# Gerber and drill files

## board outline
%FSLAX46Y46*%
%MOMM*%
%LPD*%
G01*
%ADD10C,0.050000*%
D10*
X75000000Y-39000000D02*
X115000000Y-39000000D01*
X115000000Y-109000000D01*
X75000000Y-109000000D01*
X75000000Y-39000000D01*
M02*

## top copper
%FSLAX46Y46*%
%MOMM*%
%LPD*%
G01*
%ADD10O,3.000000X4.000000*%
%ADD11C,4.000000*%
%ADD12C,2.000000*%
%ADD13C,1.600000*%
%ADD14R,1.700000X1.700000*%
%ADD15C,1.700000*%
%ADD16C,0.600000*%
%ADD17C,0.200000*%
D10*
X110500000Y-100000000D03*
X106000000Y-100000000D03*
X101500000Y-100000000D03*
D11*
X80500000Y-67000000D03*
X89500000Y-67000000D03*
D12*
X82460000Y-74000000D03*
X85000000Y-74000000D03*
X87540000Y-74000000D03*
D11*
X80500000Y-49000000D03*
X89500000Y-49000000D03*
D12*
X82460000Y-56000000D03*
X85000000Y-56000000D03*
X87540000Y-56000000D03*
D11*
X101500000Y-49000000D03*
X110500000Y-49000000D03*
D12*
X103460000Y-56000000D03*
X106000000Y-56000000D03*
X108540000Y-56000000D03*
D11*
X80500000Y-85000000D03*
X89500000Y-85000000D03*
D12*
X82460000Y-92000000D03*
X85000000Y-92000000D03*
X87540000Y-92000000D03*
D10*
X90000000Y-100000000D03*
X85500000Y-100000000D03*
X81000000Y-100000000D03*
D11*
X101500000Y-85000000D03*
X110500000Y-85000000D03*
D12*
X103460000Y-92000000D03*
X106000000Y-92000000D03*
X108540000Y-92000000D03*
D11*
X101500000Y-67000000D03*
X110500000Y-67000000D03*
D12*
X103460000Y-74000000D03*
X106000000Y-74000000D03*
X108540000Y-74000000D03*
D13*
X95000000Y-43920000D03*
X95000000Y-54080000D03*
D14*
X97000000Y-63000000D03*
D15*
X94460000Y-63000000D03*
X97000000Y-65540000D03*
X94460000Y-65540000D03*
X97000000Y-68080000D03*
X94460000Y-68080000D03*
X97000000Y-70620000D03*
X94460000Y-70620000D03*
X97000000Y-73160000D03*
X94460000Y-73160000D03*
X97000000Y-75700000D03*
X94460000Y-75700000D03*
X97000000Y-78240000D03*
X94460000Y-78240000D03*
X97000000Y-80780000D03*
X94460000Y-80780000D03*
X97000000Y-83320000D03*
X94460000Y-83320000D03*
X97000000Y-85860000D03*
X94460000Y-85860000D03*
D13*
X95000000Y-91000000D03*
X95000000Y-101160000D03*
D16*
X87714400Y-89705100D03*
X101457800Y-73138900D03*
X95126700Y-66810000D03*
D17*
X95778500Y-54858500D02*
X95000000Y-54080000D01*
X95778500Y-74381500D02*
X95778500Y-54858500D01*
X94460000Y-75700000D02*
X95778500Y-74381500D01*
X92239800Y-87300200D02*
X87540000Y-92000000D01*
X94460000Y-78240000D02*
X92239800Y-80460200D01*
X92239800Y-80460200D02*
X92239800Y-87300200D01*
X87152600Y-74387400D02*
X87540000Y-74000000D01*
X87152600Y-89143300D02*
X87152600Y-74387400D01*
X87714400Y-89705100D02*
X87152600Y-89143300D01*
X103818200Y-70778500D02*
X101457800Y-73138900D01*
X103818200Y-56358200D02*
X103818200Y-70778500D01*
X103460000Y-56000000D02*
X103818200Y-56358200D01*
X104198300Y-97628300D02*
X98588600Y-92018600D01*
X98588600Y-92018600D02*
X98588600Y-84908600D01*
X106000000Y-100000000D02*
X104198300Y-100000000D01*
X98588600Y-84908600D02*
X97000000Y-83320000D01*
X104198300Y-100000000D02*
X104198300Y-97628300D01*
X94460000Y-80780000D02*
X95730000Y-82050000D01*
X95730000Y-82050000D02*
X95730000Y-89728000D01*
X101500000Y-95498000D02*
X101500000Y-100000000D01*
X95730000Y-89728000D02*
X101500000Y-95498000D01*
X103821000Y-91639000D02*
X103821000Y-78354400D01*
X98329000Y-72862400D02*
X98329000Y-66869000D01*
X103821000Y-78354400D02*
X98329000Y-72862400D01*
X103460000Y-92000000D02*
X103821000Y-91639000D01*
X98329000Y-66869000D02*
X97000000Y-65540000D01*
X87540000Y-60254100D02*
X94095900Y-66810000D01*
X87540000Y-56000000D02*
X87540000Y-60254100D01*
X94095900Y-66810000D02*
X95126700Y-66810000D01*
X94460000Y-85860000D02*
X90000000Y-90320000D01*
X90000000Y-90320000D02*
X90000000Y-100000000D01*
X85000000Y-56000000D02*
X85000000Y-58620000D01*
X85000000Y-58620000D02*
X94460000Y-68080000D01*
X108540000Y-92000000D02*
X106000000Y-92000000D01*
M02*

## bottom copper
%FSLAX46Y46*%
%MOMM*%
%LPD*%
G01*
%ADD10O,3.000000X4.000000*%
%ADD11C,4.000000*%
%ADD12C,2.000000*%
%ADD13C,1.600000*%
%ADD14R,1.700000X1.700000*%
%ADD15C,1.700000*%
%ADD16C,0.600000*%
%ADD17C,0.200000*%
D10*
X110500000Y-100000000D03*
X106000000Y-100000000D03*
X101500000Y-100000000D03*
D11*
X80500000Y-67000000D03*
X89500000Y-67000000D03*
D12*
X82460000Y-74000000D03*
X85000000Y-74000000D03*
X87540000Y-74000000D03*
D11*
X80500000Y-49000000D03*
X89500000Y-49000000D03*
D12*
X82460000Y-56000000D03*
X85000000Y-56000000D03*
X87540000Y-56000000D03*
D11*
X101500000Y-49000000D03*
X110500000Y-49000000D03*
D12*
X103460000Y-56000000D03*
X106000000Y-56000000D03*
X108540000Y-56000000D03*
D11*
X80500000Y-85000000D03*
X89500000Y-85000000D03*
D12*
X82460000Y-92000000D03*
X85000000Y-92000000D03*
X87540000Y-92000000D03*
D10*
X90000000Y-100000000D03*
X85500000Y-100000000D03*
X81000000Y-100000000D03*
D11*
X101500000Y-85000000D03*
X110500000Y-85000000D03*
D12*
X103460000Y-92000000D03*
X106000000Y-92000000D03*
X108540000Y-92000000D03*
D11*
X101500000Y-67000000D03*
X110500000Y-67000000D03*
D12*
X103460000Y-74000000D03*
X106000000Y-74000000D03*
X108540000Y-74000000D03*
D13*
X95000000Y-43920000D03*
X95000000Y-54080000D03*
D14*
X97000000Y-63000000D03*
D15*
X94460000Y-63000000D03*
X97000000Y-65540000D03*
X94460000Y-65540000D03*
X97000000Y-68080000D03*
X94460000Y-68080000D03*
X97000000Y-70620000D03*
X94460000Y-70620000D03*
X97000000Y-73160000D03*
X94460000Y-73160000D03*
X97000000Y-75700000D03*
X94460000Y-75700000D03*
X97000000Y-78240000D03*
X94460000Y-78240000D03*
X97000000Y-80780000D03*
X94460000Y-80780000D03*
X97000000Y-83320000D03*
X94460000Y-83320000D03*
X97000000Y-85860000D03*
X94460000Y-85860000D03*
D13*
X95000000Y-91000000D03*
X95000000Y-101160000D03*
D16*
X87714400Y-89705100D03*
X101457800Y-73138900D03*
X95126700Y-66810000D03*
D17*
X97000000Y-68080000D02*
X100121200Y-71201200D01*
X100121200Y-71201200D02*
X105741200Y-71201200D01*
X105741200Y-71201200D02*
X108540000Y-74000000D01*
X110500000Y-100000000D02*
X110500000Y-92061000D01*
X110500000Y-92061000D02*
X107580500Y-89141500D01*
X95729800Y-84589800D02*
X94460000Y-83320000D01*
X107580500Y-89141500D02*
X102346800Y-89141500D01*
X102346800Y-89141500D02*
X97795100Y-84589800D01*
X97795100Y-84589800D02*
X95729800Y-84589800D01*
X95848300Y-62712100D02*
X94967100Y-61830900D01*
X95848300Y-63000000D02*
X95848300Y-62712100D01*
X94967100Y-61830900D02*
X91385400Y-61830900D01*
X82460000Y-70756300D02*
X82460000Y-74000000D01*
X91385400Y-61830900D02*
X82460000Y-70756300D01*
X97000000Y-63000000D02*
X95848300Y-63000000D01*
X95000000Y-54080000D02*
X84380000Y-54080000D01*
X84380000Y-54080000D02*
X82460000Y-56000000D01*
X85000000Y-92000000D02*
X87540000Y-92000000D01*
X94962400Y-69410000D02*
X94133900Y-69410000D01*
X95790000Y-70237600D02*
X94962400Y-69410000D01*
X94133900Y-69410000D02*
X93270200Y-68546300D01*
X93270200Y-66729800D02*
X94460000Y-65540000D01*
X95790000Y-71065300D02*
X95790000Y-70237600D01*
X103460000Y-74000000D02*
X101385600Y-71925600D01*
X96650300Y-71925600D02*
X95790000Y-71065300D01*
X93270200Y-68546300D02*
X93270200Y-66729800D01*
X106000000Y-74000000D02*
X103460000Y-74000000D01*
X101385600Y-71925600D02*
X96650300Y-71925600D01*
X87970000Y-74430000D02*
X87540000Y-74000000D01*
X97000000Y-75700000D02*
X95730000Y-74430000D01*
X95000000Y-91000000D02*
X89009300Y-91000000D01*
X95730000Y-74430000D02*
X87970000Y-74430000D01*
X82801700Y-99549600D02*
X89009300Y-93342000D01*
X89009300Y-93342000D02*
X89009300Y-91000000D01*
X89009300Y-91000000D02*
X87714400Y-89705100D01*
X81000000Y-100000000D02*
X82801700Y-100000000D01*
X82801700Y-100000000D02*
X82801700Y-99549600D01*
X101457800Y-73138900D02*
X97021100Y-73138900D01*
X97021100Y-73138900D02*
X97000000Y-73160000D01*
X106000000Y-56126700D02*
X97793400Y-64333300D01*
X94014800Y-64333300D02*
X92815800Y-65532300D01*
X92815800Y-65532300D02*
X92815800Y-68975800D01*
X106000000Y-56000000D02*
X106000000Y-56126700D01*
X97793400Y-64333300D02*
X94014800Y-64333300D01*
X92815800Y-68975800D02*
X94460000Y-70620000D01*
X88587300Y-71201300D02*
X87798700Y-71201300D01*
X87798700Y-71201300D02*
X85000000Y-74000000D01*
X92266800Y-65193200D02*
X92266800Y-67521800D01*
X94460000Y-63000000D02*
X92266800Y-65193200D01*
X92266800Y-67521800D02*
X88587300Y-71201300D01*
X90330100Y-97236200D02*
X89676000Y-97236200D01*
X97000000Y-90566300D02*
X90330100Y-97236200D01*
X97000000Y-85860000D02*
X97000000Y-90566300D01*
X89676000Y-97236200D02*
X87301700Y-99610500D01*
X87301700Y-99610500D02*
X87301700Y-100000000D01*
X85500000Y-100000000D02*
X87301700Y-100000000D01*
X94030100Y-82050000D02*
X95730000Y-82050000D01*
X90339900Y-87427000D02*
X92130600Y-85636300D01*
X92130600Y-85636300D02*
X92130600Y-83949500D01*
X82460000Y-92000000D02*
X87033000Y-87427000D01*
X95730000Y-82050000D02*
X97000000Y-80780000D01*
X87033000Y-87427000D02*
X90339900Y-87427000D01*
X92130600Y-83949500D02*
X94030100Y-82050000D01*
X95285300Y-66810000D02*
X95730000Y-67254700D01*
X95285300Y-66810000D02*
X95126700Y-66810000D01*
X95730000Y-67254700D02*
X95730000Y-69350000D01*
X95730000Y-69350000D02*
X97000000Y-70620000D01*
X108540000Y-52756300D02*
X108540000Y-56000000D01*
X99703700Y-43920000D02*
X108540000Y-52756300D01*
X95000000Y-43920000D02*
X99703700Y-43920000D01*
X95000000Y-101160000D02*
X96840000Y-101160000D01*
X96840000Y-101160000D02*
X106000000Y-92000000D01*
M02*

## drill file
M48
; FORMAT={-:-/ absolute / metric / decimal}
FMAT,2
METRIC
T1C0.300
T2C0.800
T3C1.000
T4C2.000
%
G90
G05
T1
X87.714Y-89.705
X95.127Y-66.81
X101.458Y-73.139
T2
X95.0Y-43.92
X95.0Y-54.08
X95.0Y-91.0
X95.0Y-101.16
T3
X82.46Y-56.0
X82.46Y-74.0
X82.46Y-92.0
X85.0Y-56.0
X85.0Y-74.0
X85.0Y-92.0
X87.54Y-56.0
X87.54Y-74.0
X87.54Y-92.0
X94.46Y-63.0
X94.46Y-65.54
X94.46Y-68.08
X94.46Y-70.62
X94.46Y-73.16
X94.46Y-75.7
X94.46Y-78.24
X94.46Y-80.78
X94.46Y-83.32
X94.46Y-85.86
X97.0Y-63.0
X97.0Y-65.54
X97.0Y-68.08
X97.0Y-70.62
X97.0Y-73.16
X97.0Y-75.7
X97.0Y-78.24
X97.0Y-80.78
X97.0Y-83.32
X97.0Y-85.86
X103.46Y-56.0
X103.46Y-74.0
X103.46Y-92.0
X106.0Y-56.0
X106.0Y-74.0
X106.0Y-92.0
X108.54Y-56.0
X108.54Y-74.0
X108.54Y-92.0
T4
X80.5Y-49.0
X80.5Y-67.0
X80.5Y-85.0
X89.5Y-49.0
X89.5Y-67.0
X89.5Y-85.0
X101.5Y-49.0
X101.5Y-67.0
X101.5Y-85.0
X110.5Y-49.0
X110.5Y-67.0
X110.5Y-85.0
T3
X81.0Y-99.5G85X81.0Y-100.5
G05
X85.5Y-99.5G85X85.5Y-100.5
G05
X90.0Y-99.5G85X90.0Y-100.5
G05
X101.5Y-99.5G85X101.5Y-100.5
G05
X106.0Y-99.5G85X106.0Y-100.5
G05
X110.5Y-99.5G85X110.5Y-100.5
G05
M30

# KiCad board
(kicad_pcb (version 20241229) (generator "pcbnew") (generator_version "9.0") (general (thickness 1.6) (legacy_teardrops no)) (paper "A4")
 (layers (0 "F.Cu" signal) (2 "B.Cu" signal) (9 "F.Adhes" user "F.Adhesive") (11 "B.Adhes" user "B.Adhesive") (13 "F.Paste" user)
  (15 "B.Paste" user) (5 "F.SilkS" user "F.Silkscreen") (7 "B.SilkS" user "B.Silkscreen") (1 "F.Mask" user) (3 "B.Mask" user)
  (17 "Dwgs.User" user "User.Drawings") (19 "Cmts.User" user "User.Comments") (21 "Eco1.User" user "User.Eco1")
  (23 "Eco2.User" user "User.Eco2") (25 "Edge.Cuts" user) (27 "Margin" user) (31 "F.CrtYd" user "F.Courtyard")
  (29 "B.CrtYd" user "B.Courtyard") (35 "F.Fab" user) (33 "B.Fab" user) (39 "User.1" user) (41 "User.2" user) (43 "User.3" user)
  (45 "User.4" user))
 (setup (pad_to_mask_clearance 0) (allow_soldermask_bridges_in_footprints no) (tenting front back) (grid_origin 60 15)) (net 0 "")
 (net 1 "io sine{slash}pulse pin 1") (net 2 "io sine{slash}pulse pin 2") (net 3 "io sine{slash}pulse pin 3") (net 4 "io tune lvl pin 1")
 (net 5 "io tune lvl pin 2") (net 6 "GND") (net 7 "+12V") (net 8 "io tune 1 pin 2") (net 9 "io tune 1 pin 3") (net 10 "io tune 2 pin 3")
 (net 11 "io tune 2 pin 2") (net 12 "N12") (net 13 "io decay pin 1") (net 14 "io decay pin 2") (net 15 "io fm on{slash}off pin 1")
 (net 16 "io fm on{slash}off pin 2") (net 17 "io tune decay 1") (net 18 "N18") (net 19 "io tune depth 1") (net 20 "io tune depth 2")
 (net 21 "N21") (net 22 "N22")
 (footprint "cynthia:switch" (layer "F.Cu") (at 106 100 -90)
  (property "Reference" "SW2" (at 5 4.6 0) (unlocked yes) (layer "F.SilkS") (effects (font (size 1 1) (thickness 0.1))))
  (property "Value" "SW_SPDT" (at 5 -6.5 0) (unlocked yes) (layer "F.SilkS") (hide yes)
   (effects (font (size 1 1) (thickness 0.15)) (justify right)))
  (pad "1" thru_hole oval (at 0 -4.5 270) (size 4 3) (drill oval 2 1) (layers "*.Cu" "*.Mask") (remove_unused_layers no)
   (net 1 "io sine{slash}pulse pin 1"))
  (pad "2" thru_hole oval (at 0 0 270) (size 4 3) (drill oval 2 1) (layers "*.Cu" "*.Mask") (remove_unused_layers no)
   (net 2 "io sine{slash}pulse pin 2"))
  (pad "3" thru_hole oval (at 0 4.5 270) (size 4 3) (drill oval 2 1) (layers "*.Cu" "*.Mask") (remove_unused_layers no)
   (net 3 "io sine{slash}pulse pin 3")))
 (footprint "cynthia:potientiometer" (layer "F.Cu") (at 85 67)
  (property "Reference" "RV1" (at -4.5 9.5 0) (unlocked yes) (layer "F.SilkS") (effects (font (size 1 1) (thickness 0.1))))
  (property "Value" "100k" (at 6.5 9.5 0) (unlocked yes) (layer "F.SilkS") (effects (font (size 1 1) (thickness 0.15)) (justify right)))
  (pad "" thru_hole circle (at -4.5 0) (size 4 4) (drill 2) (layers "*.Cu" "*.Mask") (remove_unused_layers no))
  (pad "" thru_hole circle (at 4.5 0) (size 4 4) (drill 2) (layers "*.Cu" "*.Mask") (remove_unused_layers no))
  (pad "1" thru_hole circle (at -2.54 7) (size 2 2) (drill 1) (layers "*.Cu" "*.Mask") (remove_unused_layers no) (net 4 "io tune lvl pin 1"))
  (pad "2" thru_hole circle (at 0 7) (size 2 2) (drill 1) (layers "*.Cu" "*.Mask") (remove_unused_layers no) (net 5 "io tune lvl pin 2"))
  (pad "3" thru_hole circle (at 2.54 7) (size 2 2) (drill 1) (layers "*.Cu" "*.Mask") (remove_unused_layers no) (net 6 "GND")))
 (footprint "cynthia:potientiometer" (layer "F.Cu") (at 85 49)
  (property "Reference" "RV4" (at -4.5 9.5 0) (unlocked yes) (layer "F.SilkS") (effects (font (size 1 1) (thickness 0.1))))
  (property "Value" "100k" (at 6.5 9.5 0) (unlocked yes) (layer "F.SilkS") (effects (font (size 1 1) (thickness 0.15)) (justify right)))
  (pad "" thru_hole circle (at -4.5 0) (size 4 4) (drill 2) (layers "*.Cu" "*.Mask") (remove_unused_layers no))
  (pad "" thru_hole circle (at 4.5 0) (size 4 4) (drill 2) (layers "*.Cu" "*.Mask") (remove_unused_layers no))
  (pad "1" thru_hole circle (at -2.54 7) (size 2 2) (drill 1) (layers "*.Cu" "*.Mask") (remove_unused_layers no) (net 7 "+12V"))
  (pad "2" thru_hole circle (at 0 7) (size 2 2) (drill 1) (layers "*.Cu" "*.Mask") (remove_unused_layers no) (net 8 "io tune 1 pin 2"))
  (pad "3" thru_hole circle (at 2.54 7) (size 2 2) (drill 1) (layers "*.Cu" "*.Mask") (remove_unused_layers no) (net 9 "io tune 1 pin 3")))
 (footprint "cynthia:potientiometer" (layer "F.Cu") (at 106 49)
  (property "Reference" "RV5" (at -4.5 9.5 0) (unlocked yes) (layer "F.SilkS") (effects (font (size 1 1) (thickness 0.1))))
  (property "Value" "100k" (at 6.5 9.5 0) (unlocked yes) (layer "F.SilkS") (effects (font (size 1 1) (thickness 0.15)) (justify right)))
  (pad "" thru_hole circle (at -4.5 0) (size 4 4) (drill 2) (layers "*.Cu" "*.Mask") (remove_unused_layers no))
  (pad "" thru_hole circle (at 4.5 0) (size 4 4) (drill 2) (layers "*.Cu" "*.Mask") (remove_unused_layers no))
  (pad "1" thru_hole circle (at -2.54 7) (size 2 2) (drill 1) (layers "*.Cu" "*.Mask") (remove_unused_layers no) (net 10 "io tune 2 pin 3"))
  (pad "2" thru_hole circle (at 0 7) (size 2 2) (drill 1) (layers "*.Cu" "*.Mask") (remove_unused_layers no) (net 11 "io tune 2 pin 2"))
  (pad "3" thru_hole circle (at 2.54 7) (size 2 2) (drill 1) (layers "*.Cu" "*.Mask") (remove_unused_layers no) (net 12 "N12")))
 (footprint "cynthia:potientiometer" (layer "F.Cu") (at 85 85)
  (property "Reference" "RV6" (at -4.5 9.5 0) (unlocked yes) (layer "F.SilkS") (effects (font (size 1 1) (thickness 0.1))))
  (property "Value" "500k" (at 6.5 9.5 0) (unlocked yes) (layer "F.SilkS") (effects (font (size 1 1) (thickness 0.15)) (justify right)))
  (pad "" thru_hole circle (at -4.5 0) (size 4 4) (drill 2) (layers "*.Cu" "*.Mask") (remove_unused_layers no))
  (pad "" thru_hole circle (at 4.5 0) (size 4 4) (drill 2) (layers "*.Cu" "*.Mask") (remove_unused_layers no))
  (pad "1" thru_hole circle (at -2.54 7) (size 2 2) (drill 1) (layers "*.Cu" "*.Mask") (remove_unused_layers no) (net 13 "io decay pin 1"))
  (pad "2" thru_hole circle (at 0 7) (size 2 2) (drill 1) (layers "*.Cu" "*.Mask") (remove_unused_layers no) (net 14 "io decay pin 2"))
  (pad "3" thru_hole circle (at 2.54 7) (size 2 2) (drill 1) (layers "*.Cu" "*.Mask") (remove_unused_layers no) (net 14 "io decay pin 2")))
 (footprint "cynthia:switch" (layer "F.Cu") (at 85.5 100 -90)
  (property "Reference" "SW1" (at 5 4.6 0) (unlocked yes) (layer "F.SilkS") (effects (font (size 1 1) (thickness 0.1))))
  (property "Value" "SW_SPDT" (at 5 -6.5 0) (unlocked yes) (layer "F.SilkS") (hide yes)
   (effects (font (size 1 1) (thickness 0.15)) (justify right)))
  (pad "1" thru_hole oval (at 0 -4.5 270) (size 4 3) (drill oval 2 1) (layers "*.Cu" "*.Mask") (remove_unused_layers no)
   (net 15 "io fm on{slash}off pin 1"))
  (pad "2" thru_hole oval (at 0 0 270) (size 4 3) (drill oval 2 1) (layers "*.Cu" "*.Mask") (remove_unused_layers no)
   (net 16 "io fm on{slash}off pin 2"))
  (pad "3" thru_hole oval (at 0 4.5 270) (size 4 3) (drill oval 2 1) (layers "*.Cu" "*.Mask") (remove_unused_layers no) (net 6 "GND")))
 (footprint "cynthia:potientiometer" (layer "F.Cu") (at 106 85)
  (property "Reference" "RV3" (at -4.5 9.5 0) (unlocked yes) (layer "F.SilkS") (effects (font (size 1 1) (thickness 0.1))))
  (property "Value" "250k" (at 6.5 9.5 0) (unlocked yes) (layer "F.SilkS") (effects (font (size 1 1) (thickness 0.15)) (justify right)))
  (pad "" thru_hole circle (at -4.5 0) (size 4 4) (drill 2) (layers "*.Cu" "*.Mask") (remove_unused_layers no))
  (pad "" thru_hole circle (at 4.5 0) (size 4 4) (drill 2) (layers "*.Cu" "*.Mask") (remove_unused_layers no))
  (pad "1" thru_hole circle (at -2.54 7) (size 2 2) (drill 1) (layers "*.Cu" "*.Mask") (remove_unused_layers no) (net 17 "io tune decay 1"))
  (pad "2" thru_hole circle (at 0 7) (size 2 2) (drill 1) (layers "*.Cu" "*.Mask") (remove_unused_layers no) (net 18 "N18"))
  (pad "3" thru_hole circle (at 2.54 7) (size 2 2) (drill 1) (layers "*.Cu" "*.Mask") (remove_unused_layers no) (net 18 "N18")))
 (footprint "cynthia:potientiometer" (layer "F.Cu") (at 106 67)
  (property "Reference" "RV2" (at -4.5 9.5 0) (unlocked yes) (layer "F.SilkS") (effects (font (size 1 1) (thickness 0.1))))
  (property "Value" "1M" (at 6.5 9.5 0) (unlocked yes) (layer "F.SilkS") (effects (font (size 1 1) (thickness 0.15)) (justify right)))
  (pad "" thru_hole circle (at -4.5 0) (size 4 4) (drill 2) (layers "*.Cu" "*.Mask") (remove_unused_layers no))
  (pad "" thru_hole circle (at 4.5 0) (size 4 4) (drill 2) (layers "*.Cu" "*.Mask") (remove_unused_layers no))
  (pad "1" thru_hole circle (at -2.54 7) (size 2 2) (drill 1) (layers "*.Cu" "*.Mask") (remove_unused_layers no) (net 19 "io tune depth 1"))
  (pad "2" thru_hole circle (at 0 7) (size 2 2) (drill 1) (layers "*.Cu" "*.Mask") (remove_unused_layers no) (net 19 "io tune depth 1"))
  (pad "3" thru_hole circle (at 2.54 7) (size 2 2) (drill 1) (layers "*.Cu" "*.Mask") (remove_unused_layers no) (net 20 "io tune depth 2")))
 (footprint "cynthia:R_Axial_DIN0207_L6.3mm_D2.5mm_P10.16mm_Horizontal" (layer "B.Cu") (at 95 43.92 -90)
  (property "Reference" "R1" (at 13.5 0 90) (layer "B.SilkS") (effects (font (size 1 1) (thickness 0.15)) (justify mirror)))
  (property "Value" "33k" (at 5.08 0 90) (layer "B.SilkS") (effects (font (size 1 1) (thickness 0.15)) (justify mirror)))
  (pad "1" thru_hole circle (at 0 0 270) (size 1.6 1.6) (drill 0.8) (layers "*.Cu" "*.Mask") (remove_unused_layers no) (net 12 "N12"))
  (pad "2" thru_hole circle (at 10.16 0 270) (size 1.6 1.6) (drill 0.8) (layers "*.Cu" "*.Mask") (remove_unused_layers no) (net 7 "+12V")))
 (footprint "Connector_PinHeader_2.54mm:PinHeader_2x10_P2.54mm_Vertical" (layer "B.Cu") (at 97 63 180)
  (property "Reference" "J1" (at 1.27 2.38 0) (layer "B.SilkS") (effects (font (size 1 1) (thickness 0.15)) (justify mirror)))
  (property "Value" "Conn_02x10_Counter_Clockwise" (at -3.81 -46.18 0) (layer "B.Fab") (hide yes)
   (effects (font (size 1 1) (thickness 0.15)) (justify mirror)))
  (pad "1" thru_hole rect (at 0 0 180) (size 1.7 1.7) (drill 1) (layers "*.Cu" "*.Mask") (remove_unused_layers no)
   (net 4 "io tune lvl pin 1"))
  (pad "2" thru_hole circle (at 2.54 0 180) (size 1.7 1.7) (drill 1) (layers "*.Cu" "*.Mask") (remove_unused_layers no)
   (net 5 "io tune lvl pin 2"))
  (pad "3" thru_hole circle (at 0 -2.54 180) (size 1.7 1.7) (drill 1) (layers "*.Cu" "*.Mask") (remove_unused_layers no)
   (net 17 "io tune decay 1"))
  (pad "4" thru_hole circle (at 2.54 -2.54 180) (size 1.7 1.7) (drill 1) (layers "*.Cu" "*.Mask") (remove_unused_layers no)
   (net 19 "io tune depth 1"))
  (pad "5" thru_hole circle (at 0 -5.08 180) (size 1.7 1.7) (drill 1) (layers "*.Cu" "*.Mask") (remove_unused_layers no)
   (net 20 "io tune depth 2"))
  (pad "6" thru_hole circle (at 2.54 -5.08 180) (size 1.7 1.7) (drill 1) (layers "*.Cu" "*.Mask") (remove_unused_layers no)
   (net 8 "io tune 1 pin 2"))
  (pad "7" thru_hole circle (at 0 -7.62 180) (size 1.7 1.7) (drill 1) (layers "*.Cu" "*.Mask") (remove_unused_layers no)
   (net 9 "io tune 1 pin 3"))
  (pad "8" thru_hole circle (at 2.54 -7.62 180) (size 1.7 1.7) (drill 1) (layers "*.Cu" "*.Mask") (remove_unused_layers no)
   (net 11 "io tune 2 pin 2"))
  (pad "9" thru_hole circle (at 0 -10.16 180) (size 1.7 1.7) (drill 1) (layers "*.Cu" "*.Mask") (remove_unused_layers no)
   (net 10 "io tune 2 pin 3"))
  (pad "10" thru_hole circle (at 2.54 -10.16 180) (size 1.7 1.7) (drill 1) (layers "*.Cu" "*.Mask") (remove_unused_layers no) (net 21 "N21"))
  (pad "11" thru_hole circle (at 0 -12.7 180) (size 1.7 1.7) (drill 1) (layers "*.Cu" "*.Mask") (remove_unused_layers no) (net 6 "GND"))
  (pad "12" thru_hole circle (at 2.54 -12.7 180) (size 1.7 1.7) (drill 1) (layers "*.Cu" "*.Mask") (remove_unused_layers no) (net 7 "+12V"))
  (pad "13" thru_hole circle (at 0 -15.24 180) (size 1.7 1.7) (drill 1) (layers "*.Cu" "*.Mask") (remove_unused_layers no) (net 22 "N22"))
  (pad "14" thru_hole circle (at 2.54 -15.24 180) (size 1.7 1.7) (drill 1) (layers "*.Cu" "*.Mask") (remove_unused_layers no)
   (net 14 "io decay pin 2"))
  (pad "15" thru_hole circle (at 0 -17.78 180) (size 1.7 1.7) (drill 1) (layers "*.Cu" "*.Mask") (remove_unused_layers no)
   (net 13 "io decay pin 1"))
  (pad "16" thru_hole circle (at 2.54 -17.78 180) (size 1.7 1.7) (drill 1) (layers "*.Cu" "*.Mask") (remove_unused_layers no)
   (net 3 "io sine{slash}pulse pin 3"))
  (pad "17" thru_hole circle (at 0 -20.32 180) (size 1.7 1.7) (drill 1) (layers "*.Cu" "*.Mask") (remove_unused_layers no)
   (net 2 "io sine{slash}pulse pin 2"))
  (pad "18" thru_hole circle (at 2.54 -20.32 180) (size 1.7 1.7) (drill 1) (layers "*.Cu" "*.Mask") (remove_unused_layers no)
   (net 1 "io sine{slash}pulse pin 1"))
  (pad "19" thru_hole circle (at 0 -22.86 180) (size 1.7 1.7) (drill 1) (layers "*.Cu" "*.Mask") (remove_unused_layers no)
   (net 16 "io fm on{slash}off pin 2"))
  (pad "20" thru_hole circle (at 2.54 -22.86 180) (size 1.7 1.7) (drill 1) (layers "*.Cu" "*.Mask") (remove_unused_layers no)
   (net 15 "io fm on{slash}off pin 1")))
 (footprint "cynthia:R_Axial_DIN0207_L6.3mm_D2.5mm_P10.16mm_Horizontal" (layer "B.Cu") (at 95 91 -90)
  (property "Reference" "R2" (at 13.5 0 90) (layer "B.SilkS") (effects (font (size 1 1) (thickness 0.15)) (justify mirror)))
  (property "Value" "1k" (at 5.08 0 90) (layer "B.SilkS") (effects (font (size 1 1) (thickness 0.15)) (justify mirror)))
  (pad "1" thru_hole circle (at 0 0 270) (size 1.6 1.6) (drill 0.8) (layers "*.Cu" "*.Mask") (remove_unused_layers no) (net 6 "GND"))
  (pad "2" thru_hole circle (at 10.16 0 270) (size 1.6 1.6) (drill 0.8) (layers "*.Cu" "*.Mask") (remove_unused_layers no) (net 18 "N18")))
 (gr_rect (start 75 39) (end 115 109) (stroke (width 0.05) (type default)) (fill no) (layer "Edge.Cuts"))
 (segment (start 97 68.08) (end 100.1212 71.2012) (width 0.2) (layer "B.Cu") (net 20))
 (segment (start 100.1212 71.2012) (end 105.7412 71.2012) (width 0.2) (layer "B.Cu") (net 20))
 (segment (start 105.7412 71.2012) (end 108.54 74) (width 0.2) (layer "B.Cu") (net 20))
 (segment (start 110.5 100) (end 110.5 92.061) (width 0.2) (layer "B.Cu") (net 1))
 (segment (start 110.5 92.061) (end 107.5805 89.1415) (width 0.2) (layer "B.Cu") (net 1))
 (segment (start 95.7298 84.5898) (end 94.46 83.32) (width 0.2) (layer "B.Cu") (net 1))
 (segment (start 107.5805 89.1415) (end 102.3468 89.1415) (width 0.2) (layer "B.Cu") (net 1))
 (segment (start 102.3468 89.1415) (end 97.7951 84.5898) (width 0.2) (layer "B.Cu") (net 1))
 (segment (start 97.7951 84.5898) (end 95.7298 84.5898) (width 0.2) (layer "B.Cu") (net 1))
 (segment (start 95.8483 62.7121) (end 94.9671 61.8309) (width 0.2) (layer "B.Cu") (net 4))
 (segment (start 95.8483 63) (end 95.8483 62.7121) (width 0.2) (layer "B.Cu") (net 4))
 (segment (start 94.9671 61.8309) (end 91.3854 61.8309) (width 0.2) (layer "B.Cu") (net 4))
 (segment (start 82.46 70.7563) (end 82.46 74) (width 0.2) (layer "B.Cu") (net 4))
 (segment (start 91.3854 61.8309) (end 82.46 70.7563) (width 0.2) (layer "B.Cu") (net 4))
 (segment (start 97 63) (end 95.8483 63) (width 0.2) (layer "B.Cu") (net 4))
 (segment (start 95.7785 54.8585) (end 95 54.08) (width 0.2) (layer "F.Cu") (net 7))
 (segment (start 95.7785 74.3815) (end 95.7785 54.8585) (width 0.2) (layer "F.Cu") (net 7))
 (segment (start 94.46 75.7) (end 95.7785 74.3815) (width 0.2) (layer "F.Cu") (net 7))
 (segment (start 95 54.08) (end 84.38 54.08) (width 0.2) (layer "B.Cu") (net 7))
 (segment (start 84.38 54.08) (end 82.46 56) (width 0.2) (layer "B.Cu") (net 7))
 (segment (start 92.2398 87.3002) (end 87.54 92) (width 0.2) (layer "F.Cu") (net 14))
 (segment (start 94.46 78.24) (end 92.2398 80.4602) (width 0.2) (layer "F.Cu") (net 14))
 (segment (start 92.2398 80.4602) (end 92.2398 87.3002) (width 0.2) (layer "F.Cu") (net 14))
 (segment (start 85 92) (end 87.54 92) (width 0.2) (layer "B.Cu") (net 14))
 (segment (start 94.9624 69.41) (end 94.1339 69.41) (width 0.2) (layer "B.Cu") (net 19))
 (segment (start 95.79 70.2376) (end 94.9624 69.41) (width 0.2) (layer "B.Cu") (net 19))
 (segment (start 94.1339 69.41) (end 93.2702 68.5463) (width 0.2) (layer "B.Cu") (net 19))
 (segment (start 93.2702 66.7298) (end 94.46 65.54) (width 0.2) (layer "B.Cu") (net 19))
 (segment (start 95.79 71.0653) (end 95.79 70.2376) (width 0.2) (layer "B.Cu") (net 19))
 (segment (start 103.46 74) (end 101.3856 71.9256) (width 0.2) (layer "B.Cu") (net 19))
 (segment (start 96.6503 71.9256) (end 95.79 71.0653) (width 0.2) (layer "B.Cu") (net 19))
 (segment (start 93.2702 68.5463) (end 93.2702 66.7298) (width 0.2) (layer "B.Cu") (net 19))
 (segment (start 106 74) (end 103.46 74) (width 0.2) (layer "B.Cu") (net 19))
 (segment (start 101.3856 71.9256) (end 96.6503 71.9256) (width 0.2) (layer "B.Cu") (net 19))
 (segment (start 87.1526 74.3874) (end 87.54 74) (width 0.2) (layer "F.Cu") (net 6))
 (segment (start 87.1526 89.1433) (end 87.1526 74.3874) (width 0.2) (layer "F.Cu") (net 6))
 (segment (start 87.7144 89.7051) (end 87.1526 89.1433) (width 0.2) (layer "F.Cu") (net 6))
 (via (at 87.7144 89.7051) (size 0.6) (drill 0.3) (layers "F.Cu" "B.Cu") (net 6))
 (segment (start 87.97 74.43) (end 87.54 74) (width 0.2) (layer "B.Cu") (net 6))
 (segment (start 97 75.7) (end 95.73 74.43) (width 0.2) (layer "B.Cu") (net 6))
 (segment (start 95 91) (end 89.0093 91) (width 0.2) (layer "B.Cu") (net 6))
 (segment (start 95.73 74.43) (end 87.97 74.43) (width 0.2) (layer "B.Cu") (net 6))
 (segment (start 82.8017 99.5496) (end 89.0093 93.342) (width 0.2) (layer "B.Cu") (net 6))
 (segment (start 89.0093 93.342) (end 89.0093 91) (width 0.2) (layer "B.Cu") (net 6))
 (segment (start 89.0093 91) (end 87.7144 89.7051) (width 0.2) (layer "B.Cu") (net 6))
 (segment (start 81 100) (end 82.8017 100) (width 0.2) (layer "B.Cu") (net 6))
 (segment (start 82.8017 100) (end 82.8017 99.5496) (width 0.2) (layer "B.Cu") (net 6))
 (segment (start 103.8182 70.7785) (end 101.4578 73.1389) (width 0.2) (layer "F.Cu") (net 10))
 (segment (start 103.8182 56.3582) (end 103.8182 70.7785) (width 0.2) (layer "F.Cu") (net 10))
 (segment (start 103.46 56) (end 103.8182 56.3582) (width 0.2) (layer "F.Cu") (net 10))
 (via (at 101.4578 73.1389) (size 0.6) (drill 0.3) (layers "F.Cu" "B.Cu") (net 10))
 (segment (start 101.4578 73.1389) (end 97.0211 73.1389) (width 0.2) (layer "B.Cu") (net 10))
 (segment (start 97.0211 73.1389) (end 97 73.16) (width 0.2) (layer "B.Cu") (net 10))
 (segment (start 106 56.1267) (end 97.7934 64.3333) (width 0.2) (layer "B.Cu") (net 11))
 (segment (start 94.0148 64.3333) (end 92.8158 65.5323) (width 0.2) (layer "B.Cu") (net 11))
 (segment (start 92.8158 65.5323) (end 92.8158 68.9758) (width 0.2) (layer "B.Cu") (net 11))
 (segment (start 106 56) (end 106 56.1267) (width 0.2) (layer "B.Cu") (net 11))
 (segment (start 97.7934 64.3333) (end 94.0148 64.3333) (width 0.2) (layer "B.Cu") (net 11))
 (segment (start 92.8158 68.9758) (end 94.46 70.62) (width 0.2) (layer "B.Cu") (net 11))
 (segment (start 88.5873 71.2013) (end 87.7987 71.2013) (width 0.2) (layer "B.Cu") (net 5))
 (segment (start 87.7987 71.2013) (end 85 74) (width 0.2) (layer "B.Cu") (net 5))
 (segment (start 92.2668 65.1932) (end 92.2668 67.5218) (width 0.2) (layer "B.Cu") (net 5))
 (segment (start 94.46 63) (end 92.2668 65.1932) (width 0.2) (layer "B.Cu") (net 5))
 (segment (start 92.2668 67.5218) (end 88.5873 71.2013) (width 0.2) (layer "B.Cu") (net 5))
 (segment (start 90.3301 97.2362) (end 89.676 97.2362) (width 0.2) (layer "B.Cu") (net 16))
 (segment (start 97 90.5663) (end 90.3301 97.2362) (width 0.2) (layer "B.Cu") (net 16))
 (segment (start 97 85.86) (end 97 90.5663) (width 0.2) (layer "B.Cu") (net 16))
 (segment (start 89.676 97.2362) (end 87.3017 99.6105) (width 0.2) (layer "B.Cu") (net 16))
 (segment (start 87.3017 99.6105) (end 87.3017 100) (width 0.2) (layer "B.Cu") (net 16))
 (segment (start 85.5 100) (end 87.3017 100) (width 0.2) (layer "B.Cu") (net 16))
 (segment (start 104.1983 97.6283) (end 98.5886 92.0186) (width 0.2) (layer "F.Cu") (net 2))
 (segment (start 98.5886 92.0186) (end 98.5886 84.9086) (width 0.2) (layer "F.Cu") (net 2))
 (segment (start 106 100) (end 104.1983 100) (width 0.2) (layer "F.Cu") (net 2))
 (segment (start 98.5886 84.9086) (end 97 83.32) (width 0.2) (layer "F.Cu") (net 2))
 (segment (start 104.1983 100) (end 104.1983 97.6283) (width 0.2) (layer "F.Cu") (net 2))
 (segment (start 94.46 80.78) (end 95.73 82.05) (width 0.2) (layer "F.Cu") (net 3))
 (segment (start 95.73 82.05) (end 95.73 89.728) (width 0.2) (layer "F.Cu") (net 3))
 (segment (start 101.5 95.498) (end 101.5 100) (width 0.2) (layer "F.Cu") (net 3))
 (segment (start 95.73 89.728) (end 101.5 95.498) (width 0.2) (layer "F.Cu") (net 3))
 (segment (start 103.821 91.639) (end 103.821 78.3544) (width 0.2) (layer "F.Cu") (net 17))
 (segment (start 98.329 72.8624) (end 98.329 66.869) (width 0.2) (layer "F.Cu") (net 17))
 (segment (start 103.821 78.3544) (end 98.329 72.8624) (width 0.2) (layer "F.Cu") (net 17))
 (segment (start 103.46 92) (end 103.821 91.639) (width 0.2) (layer "F.Cu") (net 17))
 (segment (start 98.329 66.869) (end 97 65.54) (width 0.2) (layer "F.Cu") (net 17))
 (segment (start 94.0301 82.05) (end 95.73 82.05) (width 0.2) (layer "B.Cu") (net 13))
 (segment (start 90.3399 87.427) (end 92.1306 85.6363) (width 0.2) (layer "B.Cu") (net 13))
 (segment (start 92.1306 85.6363) (end 92.1306 83.9495) (width 0.2) (layer "B.Cu") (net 13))
 (segment (start 82.46 92) (end 87.033 87.427) (width 0.2) (layer "B.Cu") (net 13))
 (segment (start 95.73 82.05) (end 97 80.78) (width 0.2) (layer "B.Cu") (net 13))
 (segment (start 87.033 87.427) (end 90.3399 87.427) (width 0.2) (layer "B.Cu") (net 13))
 (segment (start 92.1306 83.9495) (end 94.0301 82.05) (width 0.2) (layer "B.Cu") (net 13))
 (segment (start 87.54 60.2541) (end 94.0959 66.81) (width 0.2) (layer "F.Cu") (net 9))
 (segment (start 87.54 56) (end 87.54 60.2541) (width 0.2) (layer "F.Cu") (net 9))
 (segment (start 94.0959 66.81) (end 95.1267 66.81) (width 0.2) (layer "F.Cu") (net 9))
 (via (at 95.1267 66.81) (size 0.6) (drill 0.3) (layers "F.Cu" "B.Cu") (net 9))
 (segment (start 95.2853 66.81) (end 95.73 67.2547) (width 0.2) (layer "B.Cu") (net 9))
 (segment (start 95.2853 66.81) (end 95.1267 66.81) (width 0.2) (layer "B.Cu") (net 9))
 (segment (start 95.73 67.2547) (end 95.73 69.35) (width 0.2) (layer "B.Cu") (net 9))
 (segment (start 95.73 69.35) (end 97 70.62) (width 0.2) (layer "B.Cu") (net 9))
 (segment (start 94.46 85.86) (end 90 90.32) (width 0.2) (layer "F.Cu") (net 15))
 (segment (start 90 90.32) (end 90 100) (width 0.2) (layer "F.Cu") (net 15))
 (segment (start 85 56) (end 85 58.62) (width 0.2) (layer "F.Cu") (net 8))
 (segment (start 85 58.62) (end 94.46 68.08) (width 0.2) (layer "F.Cu") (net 8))
 (segment (start 108.54 52.7563) (end 108.54 56) (width 0.2) (layer "B.Cu") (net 12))
 (segment (start 99.7037 43.92) (end 108.54 52.7563) (width 0.2) (layer "B.Cu") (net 12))
 (segment (start 95 43.92) (end 99.7037 43.92) (width 0.2) (layer "B.Cu") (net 12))
 (segment (start 108.54 92) (end 106 92) (width 0.2) (layer "F.Cu") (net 18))
 (segment (start 95 101.16) (end 96.84 101.16) (width 0.2) (layer "B.Cu") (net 18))
 (segment (start 96.84 101.16) (end 106 92) (width 0.2) (layer "B.Cu") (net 18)))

